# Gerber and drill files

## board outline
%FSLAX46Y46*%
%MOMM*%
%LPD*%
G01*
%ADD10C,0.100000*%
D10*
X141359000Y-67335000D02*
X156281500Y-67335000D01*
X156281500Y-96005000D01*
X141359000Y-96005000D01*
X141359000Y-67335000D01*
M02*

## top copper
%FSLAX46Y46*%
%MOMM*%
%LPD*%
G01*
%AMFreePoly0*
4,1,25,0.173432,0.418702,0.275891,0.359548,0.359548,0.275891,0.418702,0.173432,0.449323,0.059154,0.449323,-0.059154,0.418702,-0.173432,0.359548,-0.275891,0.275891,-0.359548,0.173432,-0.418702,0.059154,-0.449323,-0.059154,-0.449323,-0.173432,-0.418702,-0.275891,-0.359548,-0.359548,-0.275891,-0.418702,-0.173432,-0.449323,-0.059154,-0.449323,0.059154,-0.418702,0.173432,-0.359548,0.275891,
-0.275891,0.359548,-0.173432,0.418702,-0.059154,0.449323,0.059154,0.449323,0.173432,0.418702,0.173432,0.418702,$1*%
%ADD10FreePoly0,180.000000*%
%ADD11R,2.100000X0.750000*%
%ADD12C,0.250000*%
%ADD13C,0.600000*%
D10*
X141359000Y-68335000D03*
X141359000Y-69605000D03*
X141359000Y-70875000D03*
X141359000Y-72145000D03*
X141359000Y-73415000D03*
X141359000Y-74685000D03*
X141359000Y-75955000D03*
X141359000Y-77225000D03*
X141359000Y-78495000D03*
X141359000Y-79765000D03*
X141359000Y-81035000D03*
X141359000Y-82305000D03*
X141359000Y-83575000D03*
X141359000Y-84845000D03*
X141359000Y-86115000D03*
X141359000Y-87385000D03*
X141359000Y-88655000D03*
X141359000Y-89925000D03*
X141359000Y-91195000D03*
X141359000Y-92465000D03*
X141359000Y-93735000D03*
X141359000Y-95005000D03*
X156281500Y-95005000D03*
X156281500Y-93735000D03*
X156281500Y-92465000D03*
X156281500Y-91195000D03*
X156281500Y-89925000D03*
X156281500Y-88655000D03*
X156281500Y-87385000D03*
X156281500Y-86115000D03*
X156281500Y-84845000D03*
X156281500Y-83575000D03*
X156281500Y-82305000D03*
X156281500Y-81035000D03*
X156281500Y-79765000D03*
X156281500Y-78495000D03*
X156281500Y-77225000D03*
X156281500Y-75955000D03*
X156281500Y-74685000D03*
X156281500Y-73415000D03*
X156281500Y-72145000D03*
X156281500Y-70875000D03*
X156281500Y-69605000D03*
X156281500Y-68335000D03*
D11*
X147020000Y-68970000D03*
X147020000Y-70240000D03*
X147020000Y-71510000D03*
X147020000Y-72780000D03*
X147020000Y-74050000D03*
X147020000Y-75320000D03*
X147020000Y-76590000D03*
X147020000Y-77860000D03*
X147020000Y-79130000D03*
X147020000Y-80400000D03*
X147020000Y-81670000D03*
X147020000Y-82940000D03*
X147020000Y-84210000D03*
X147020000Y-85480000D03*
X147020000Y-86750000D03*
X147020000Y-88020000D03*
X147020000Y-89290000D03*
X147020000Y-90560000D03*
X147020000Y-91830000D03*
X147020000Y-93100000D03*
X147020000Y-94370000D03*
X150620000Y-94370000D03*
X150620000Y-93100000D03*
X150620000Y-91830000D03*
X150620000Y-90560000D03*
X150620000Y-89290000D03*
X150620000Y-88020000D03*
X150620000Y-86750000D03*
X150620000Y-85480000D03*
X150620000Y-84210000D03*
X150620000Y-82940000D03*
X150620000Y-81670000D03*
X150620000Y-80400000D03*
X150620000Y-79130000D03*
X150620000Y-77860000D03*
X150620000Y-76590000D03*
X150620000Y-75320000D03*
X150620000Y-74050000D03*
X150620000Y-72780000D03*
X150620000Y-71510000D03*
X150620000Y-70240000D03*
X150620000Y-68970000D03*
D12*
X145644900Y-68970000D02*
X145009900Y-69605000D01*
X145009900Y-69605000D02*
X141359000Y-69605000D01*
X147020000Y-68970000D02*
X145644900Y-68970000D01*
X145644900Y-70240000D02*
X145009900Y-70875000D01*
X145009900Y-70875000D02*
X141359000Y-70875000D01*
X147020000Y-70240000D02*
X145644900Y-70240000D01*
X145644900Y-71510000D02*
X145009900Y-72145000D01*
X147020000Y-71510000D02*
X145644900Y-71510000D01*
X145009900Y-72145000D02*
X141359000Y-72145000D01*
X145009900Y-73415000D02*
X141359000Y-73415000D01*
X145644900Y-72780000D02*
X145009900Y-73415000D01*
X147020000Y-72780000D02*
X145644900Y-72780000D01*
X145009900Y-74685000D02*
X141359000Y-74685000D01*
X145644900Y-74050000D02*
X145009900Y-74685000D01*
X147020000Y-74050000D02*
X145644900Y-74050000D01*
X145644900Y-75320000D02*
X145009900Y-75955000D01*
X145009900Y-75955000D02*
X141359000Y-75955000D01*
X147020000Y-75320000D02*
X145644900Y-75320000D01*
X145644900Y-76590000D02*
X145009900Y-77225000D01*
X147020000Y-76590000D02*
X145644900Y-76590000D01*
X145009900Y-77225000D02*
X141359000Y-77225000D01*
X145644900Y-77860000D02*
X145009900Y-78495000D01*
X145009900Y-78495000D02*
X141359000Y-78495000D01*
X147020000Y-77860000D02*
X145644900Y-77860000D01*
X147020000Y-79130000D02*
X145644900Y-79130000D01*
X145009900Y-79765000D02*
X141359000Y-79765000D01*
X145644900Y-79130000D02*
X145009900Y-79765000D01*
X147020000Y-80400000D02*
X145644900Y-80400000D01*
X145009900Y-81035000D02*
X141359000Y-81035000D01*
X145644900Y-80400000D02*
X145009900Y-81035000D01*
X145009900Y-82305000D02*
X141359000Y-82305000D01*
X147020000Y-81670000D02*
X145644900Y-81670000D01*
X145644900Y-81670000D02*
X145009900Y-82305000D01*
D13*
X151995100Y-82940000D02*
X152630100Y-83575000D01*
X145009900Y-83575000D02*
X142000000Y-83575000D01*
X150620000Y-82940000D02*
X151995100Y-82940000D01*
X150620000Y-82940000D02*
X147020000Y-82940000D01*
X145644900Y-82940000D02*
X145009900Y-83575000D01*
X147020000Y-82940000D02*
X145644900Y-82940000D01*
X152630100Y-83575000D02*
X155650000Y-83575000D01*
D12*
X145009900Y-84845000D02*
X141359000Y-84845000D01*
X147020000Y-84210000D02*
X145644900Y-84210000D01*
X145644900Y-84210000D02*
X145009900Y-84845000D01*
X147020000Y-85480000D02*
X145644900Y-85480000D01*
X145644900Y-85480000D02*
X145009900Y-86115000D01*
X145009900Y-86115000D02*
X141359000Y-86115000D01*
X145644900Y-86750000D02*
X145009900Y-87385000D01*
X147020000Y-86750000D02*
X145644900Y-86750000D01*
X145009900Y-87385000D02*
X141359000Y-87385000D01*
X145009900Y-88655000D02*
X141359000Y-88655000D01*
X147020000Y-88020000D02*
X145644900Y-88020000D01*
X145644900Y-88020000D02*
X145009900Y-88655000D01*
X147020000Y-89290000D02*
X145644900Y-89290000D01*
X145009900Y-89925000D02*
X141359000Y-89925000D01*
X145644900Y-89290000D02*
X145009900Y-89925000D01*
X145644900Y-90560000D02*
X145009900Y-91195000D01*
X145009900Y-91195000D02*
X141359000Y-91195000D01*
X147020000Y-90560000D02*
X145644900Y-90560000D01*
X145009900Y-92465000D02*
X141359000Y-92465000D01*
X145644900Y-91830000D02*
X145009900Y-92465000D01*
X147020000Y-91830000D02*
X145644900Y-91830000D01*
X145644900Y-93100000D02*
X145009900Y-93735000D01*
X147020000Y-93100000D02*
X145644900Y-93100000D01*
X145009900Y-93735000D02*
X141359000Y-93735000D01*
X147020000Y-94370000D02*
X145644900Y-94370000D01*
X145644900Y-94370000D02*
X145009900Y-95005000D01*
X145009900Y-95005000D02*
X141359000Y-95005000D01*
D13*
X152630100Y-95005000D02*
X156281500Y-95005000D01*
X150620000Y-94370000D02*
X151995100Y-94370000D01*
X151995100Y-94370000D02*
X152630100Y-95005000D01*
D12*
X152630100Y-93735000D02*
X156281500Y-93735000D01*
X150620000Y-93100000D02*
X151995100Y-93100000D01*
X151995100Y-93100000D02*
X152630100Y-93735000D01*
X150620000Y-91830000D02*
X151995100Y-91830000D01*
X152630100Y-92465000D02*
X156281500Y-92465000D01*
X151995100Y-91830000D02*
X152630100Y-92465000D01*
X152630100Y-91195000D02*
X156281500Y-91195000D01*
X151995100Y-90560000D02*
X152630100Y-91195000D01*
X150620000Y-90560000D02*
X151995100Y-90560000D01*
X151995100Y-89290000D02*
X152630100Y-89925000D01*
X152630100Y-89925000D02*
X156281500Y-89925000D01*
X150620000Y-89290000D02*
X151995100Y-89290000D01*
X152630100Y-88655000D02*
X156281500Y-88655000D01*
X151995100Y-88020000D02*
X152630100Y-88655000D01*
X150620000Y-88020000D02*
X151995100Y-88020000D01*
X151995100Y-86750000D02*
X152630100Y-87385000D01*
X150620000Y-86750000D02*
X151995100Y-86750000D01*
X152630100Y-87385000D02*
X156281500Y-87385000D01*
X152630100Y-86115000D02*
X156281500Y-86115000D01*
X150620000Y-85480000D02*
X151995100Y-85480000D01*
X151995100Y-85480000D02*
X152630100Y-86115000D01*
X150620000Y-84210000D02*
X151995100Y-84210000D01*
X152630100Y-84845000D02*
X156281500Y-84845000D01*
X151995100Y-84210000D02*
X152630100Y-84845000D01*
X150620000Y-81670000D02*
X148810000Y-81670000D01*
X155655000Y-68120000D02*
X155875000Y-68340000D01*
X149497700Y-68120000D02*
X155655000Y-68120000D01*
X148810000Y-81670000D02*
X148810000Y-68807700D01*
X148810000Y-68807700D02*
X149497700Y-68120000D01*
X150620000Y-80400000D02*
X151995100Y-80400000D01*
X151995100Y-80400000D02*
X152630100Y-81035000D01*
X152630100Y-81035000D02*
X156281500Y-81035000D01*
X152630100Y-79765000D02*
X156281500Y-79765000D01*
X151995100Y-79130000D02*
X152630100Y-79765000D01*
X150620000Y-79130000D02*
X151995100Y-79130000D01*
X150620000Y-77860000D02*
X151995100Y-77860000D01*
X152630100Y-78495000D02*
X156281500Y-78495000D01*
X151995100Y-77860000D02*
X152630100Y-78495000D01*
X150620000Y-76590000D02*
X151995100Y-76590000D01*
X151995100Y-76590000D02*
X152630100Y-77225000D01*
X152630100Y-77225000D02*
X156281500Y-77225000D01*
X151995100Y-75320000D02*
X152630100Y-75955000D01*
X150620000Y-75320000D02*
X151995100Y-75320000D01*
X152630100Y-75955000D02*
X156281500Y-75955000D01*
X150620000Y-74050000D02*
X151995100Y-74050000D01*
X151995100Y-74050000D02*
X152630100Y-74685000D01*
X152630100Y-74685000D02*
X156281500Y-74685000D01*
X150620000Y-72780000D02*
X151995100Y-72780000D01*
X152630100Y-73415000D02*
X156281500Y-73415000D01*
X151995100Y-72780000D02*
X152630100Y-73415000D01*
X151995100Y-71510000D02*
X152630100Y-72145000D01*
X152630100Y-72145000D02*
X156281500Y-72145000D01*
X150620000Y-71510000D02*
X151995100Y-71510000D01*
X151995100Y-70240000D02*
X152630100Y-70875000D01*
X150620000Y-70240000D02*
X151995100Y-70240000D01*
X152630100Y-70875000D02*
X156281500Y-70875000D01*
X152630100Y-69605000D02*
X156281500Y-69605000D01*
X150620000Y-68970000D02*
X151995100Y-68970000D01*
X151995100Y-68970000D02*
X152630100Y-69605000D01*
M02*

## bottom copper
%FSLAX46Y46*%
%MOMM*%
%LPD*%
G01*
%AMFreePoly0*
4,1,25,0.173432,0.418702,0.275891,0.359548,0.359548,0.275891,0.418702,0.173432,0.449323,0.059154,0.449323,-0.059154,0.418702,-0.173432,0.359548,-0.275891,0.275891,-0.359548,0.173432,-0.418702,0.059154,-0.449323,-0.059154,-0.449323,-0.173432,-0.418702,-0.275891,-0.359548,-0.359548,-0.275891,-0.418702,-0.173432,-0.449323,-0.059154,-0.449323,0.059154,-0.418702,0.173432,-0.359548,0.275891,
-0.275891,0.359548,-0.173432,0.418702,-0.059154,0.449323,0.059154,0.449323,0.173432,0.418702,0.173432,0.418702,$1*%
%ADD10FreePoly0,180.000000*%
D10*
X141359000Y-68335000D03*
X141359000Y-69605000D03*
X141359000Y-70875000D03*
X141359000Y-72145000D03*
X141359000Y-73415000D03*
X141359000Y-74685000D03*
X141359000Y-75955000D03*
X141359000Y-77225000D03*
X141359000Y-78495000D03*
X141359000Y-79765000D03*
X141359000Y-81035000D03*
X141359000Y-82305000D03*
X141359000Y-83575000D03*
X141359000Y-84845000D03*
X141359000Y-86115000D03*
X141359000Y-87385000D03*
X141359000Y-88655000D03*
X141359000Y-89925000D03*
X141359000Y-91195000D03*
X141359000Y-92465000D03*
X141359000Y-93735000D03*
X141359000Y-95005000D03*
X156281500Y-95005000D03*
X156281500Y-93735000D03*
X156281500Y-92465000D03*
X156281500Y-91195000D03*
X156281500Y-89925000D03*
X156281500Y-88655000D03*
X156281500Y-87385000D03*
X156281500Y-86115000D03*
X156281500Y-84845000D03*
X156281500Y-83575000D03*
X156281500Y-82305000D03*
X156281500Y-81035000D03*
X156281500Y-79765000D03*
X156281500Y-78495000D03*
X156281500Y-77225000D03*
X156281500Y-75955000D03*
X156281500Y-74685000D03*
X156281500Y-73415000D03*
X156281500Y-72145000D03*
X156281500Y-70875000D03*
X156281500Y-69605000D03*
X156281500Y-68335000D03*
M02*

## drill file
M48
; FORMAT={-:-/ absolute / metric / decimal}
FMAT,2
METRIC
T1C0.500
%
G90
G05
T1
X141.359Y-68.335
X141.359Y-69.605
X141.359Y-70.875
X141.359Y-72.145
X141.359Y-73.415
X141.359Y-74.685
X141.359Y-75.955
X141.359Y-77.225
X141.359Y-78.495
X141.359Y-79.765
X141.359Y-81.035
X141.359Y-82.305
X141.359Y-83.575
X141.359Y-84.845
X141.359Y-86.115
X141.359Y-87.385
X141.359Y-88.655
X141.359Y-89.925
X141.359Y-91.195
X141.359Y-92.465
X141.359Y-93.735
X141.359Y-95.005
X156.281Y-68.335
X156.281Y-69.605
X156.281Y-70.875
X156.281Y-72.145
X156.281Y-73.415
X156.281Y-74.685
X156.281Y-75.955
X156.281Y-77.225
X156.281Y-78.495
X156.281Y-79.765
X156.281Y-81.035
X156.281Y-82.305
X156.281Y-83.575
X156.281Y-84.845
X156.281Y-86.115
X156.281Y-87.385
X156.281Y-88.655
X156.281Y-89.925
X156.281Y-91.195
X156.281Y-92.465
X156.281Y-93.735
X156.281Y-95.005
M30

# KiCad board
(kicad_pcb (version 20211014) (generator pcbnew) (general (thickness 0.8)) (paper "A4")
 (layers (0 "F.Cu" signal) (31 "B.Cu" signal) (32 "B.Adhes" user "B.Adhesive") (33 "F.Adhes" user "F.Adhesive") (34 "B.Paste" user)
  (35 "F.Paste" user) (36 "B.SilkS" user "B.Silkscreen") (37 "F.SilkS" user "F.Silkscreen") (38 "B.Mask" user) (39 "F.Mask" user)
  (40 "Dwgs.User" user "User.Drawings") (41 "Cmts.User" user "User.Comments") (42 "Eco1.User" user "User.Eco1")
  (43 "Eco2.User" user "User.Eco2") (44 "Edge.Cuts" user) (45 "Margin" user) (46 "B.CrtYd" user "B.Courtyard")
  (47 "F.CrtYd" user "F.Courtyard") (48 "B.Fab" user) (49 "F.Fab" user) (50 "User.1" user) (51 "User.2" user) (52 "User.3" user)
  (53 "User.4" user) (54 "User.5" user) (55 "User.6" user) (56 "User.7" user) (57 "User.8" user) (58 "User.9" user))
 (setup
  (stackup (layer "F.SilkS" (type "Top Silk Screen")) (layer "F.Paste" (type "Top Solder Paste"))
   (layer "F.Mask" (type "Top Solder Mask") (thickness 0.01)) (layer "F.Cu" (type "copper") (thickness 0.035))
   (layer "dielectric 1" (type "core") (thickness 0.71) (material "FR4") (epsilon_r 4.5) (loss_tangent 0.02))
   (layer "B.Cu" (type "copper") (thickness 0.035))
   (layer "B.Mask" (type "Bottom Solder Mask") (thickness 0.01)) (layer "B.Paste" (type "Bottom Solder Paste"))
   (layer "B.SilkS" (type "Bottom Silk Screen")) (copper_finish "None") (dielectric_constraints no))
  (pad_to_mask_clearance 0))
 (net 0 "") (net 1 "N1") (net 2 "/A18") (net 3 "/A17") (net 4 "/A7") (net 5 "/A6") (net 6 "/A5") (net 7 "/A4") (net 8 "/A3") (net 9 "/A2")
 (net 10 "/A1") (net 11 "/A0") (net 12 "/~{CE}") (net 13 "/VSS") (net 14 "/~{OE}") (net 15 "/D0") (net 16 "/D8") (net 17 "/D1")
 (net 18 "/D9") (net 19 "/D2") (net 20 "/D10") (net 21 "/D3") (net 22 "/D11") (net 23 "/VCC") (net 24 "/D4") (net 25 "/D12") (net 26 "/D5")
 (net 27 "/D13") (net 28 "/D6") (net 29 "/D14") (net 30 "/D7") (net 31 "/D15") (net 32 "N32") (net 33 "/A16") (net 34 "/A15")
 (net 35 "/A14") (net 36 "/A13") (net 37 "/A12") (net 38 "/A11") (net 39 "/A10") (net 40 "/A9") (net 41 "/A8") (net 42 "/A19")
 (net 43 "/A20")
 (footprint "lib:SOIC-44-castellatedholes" (layer "F.Cu") (at 148.82 81.67)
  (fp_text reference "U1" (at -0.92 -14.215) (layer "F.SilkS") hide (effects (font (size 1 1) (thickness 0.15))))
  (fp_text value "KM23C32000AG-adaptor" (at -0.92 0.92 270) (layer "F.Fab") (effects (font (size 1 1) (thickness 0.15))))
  (pad "1" thru_hole custom (at -7.461 -13.335 180) (size 0.9064 0.9064) (drill 0.5) (layers *.Cu *.Mask) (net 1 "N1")
   (solder_mask_margin 0.0762) (options (clearance outline) (anchor circle)) (primitives))
  (pad "2" thru_hole custom (at -7.461 -12.065 180) (size 0.9064 0.9064) (drill 0.5) (layers *.Cu *.Mask) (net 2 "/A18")
   (solder_mask_margin 0.0762) (options (clearance outline) (anchor circle)) (primitives))
  (pad "3" thru_hole custom (at -7.461 -10.795 180) (size 0.9064 0.9064) (drill 0.5) (layers *.Cu *.Mask) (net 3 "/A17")
   (solder_mask_margin 0.0762) (options (clearance outline) (anchor circle)) (primitives))
  (pad "4" thru_hole custom (at -7.461 -9.525 180) (size 0.9064 0.9064) (drill 0.5) (layers *.Cu *.Mask) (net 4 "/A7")
   (solder_mask_margin 0.0762) (options (clearance outline) (anchor circle)) (primitives))
  (pad "5" thru_hole custom (at -7.461 -8.255 180) (size 0.9064 0.9064) (drill 0.5) (layers *.Cu *.Mask) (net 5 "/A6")
   (solder_mask_margin 0.0762) (options (clearance outline) (anchor circle)) (primitives))
  (pad "6" thru_hole custom (at -7.461 -6.985 180) (size 0.9064 0.9064) (drill 0.5) (layers *.Cu *.Mask) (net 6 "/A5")
   (solder_mask_margin 0.0762) (options (clearance outline) (anchor circle)) (primitives))
  (pad "7" thru_hole custom (at -7.461 -5.715 180) (size 0.9064 0.9064) (drill 0.5) (layers *.Cu *.Mask) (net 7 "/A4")
   (solder_mask_margin 0.0762) (options (clearance outline) (anchor circle)) (primitives))
  (pad "8" thru_hole custom (at -7.461 -4.445 180) (size 0.9064 0.9064) (drill 0.5) (layers *.Cu *.Mask) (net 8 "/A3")
   (solder_mask_margin 0.0762) (options (clearance outline) (anchor circle)) (primitives))
  (pad "9" thru_hole custom (at -7.461 -3.175 180) (size 0.9064 0.9064) (drill 0.5) (layers *.Cu *.Mask) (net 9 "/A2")
   (solder_mask_margin 0.0762) (options (clearance outline) (anchor circle)) (primitives))
  (pad "10" thru_hole custom (at -7.461 -1.905 180) (size 0.9064 0.9064) (drill 0.5) (layers *.Cu *.Mask) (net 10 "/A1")
   (solder_mask_margin 0.0762) (options (clearance outline) (anchor circle)) (primitives))
  (pad "11" thru_hole custom (at -7.461 -0.635 180) (size 0.9064 0.9064) (drill 0.5) (layers *.Cu *.Mask) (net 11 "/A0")
   (solder_mask_margin 0.0762) (options (clearance outline) (anchor circle)) (primitives))
  (pad "12" thru_hole custom (at -7.461 0.635 180) (size 0.9064 0.9064) (drill 0.5) (layers *.Cu *.Mask) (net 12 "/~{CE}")
   (solder_mask_margin 0.0762) (options (clearance outline) (anchor circle)) (primitives))
  (pad "13" thru_hole custom (at -7.461 1.905 180) (size 0.9064 0.9064) (drill 0.5) (layers *.Cu *.Mask) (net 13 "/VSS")
   (solder_mask_margin 0.0762) (options (clearance outline) (anchor circle)) (primitives))
  (pad "14" thru_hole custom (at -7.461 3.175 180) (size 0.9064 0.9064) (drill 0.5) (layers *.Cu *.Mask) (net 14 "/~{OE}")
   (solder_mask_margin 0.0762) (options (clearance outline) (anchor circle)) (primitives))
  (pad "15" thru_hole custom (at -7.461 4.445 180) (size 0.9064 0.9064) (drill 0.5) (layers *.Cu *.Mask) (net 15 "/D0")
   (solder_mask_margin 0.0762) (options (clearance outline) (anchor circle)) (primitives))
  (pad "16" thru_hole custom (at -7.461 5.715 180) (size 0.9064 0.9064) (drill 0.5) (layers *.Cu *.Mask) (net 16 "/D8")
   (solder_mask_margin 0.0762) (options (clearance outline) (anchor circle)) (primitives))
  (pad "17" thru_hole custom (at -7.461 6.985 180) (size 0.9064 0.9064) (drill 0.5) (layers *.Cu *.Mask) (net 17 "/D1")
   (solder_mask_margin 0.0762) (options (clearance outline) (anchor circle)) (primitives))
  (pad "18" thru_hole custom (at -7.461 8.255 180) (size 0.9064 0.9064) (drill 0.5) (layers *.Cu *.Mask) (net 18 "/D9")
   (solder_mask_margin 0.0762) (options (clearance outline) (anchor circle)) (primitives))
  (pad "19" thru_hole custom (at -7.461 9.525 180) (size 0.9064 0.9064) (drill 0.5) (layers *.Cu *.Mask) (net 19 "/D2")
   (solder_mask_margin 0.0762) (options (clearance outline) (anchor circle)) (primitives))
  (pad "20" thru_hole custom (at -7.461 10.795 180) (size 0.9064 0.9064) (drill 0.5) (layers *.Cu *.Mask) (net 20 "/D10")
   (solder_mask_margin 0.0762) (options (clearance outline) (anchor circle)) (primitives))
  (pad "21" thru_hole custom (at -7.461 12.065 180) (size 0.9064 0.9064) (drill 0.5) (layers *.Cu *.Mask) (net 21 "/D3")
   (solder_mask_margin 0.0762) (options (clearance outline) (anchor circle)) (primitives))
  (pad "22" thru_hole custom (at -7.461 13.335 180) (size 0.9064 0.9064) (drill 0.5) (layers *.Cu *.Mask) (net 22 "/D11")
   (solder_mask_margin 0.0762) (options (clearance outline) (anchor circle)) (primitives))
  (pad "23" thru_hole custom (at 7.4615 13.335 180) (size 0.9064 0.9064) (drill 0.5) (layers *.Cu *.Mask) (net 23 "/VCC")
   (solder_mask_margin 0.0762) (options (clearance outline) (anchor circle)) (primitives))
  (pad "24" thru_hole custom (at 7.4615 12.065 180) (size 0.9064 0.9064) (drill 0.5) (layers *.Cu *.Mask) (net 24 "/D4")
   (solder_mask_margin 0.0762) (options (clearance outline) (anchor circle)) (primitives))
  (pad "25" thru_hole custom (at 7.4615 10.795 180) (size 0.9064 0.9064) (drill 0.5) (layers *.Cu *.Mask) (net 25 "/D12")
   (solder_mask_margin 0.0762) (options (clearance outline) (anchor circle)) (primitives))
  (pad "26" thru_hole custom (at 7.4615 9.525 180) (size 0.9064 0.9064) (drill 0.5) (layers *.Cu *.Mask) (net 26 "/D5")
   (solder_mask_margin 0.0762) (options (clearance outline) (anchor circle)) (primitives))
  (pad "27" thru_hole custom (at 7.4615 8.255 180) (size 0.9064 0.9064) (drill 0.5) (layers *.Cu *.Mask) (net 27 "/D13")
   (solder_mask_margin 0.0762) (options (clearance outline) (anchor circle)) (primitives))
  (pad "28" thru_hole custom (at 7.4615 6.985 180) (size 0.9064 0.9064) (drill 0.5) (layers *.Cu *.Mask) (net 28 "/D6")
   (solder_mask_margin 0.0762) (options (clearance outline) (anchor circle)) (primitives))
  (pad "29" thru_hole custom (at 7.4615 5.715 180) (size 0.9064 0.9064) (drill 0.5) (layers *.Cu *.Mask) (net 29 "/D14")
   (solder_mask_margin 0.0762) (options (clearance outline) (anchor circle)) (primitives))
  (pad "30" thru_hole custom (at 7.4615 4.445 180) (size 0.9064 0.9064) (drill 0.5) (layers *.Cu *.Mask) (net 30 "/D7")
   (solder_mask_margin 0.0762) (options (clearance outline) (anchor circle)) (primitives))
  (pad "31" thru_hole custom (at 7.4615 3.175 180) (size 0.9064 0.9064) (drill 0.5) (layers *.Cu *.Mask) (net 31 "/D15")
   (solder_mask_margin 0.0762) (options (clearance outline) (anchor circle)) (primitives))
  (pad "32" thru_hole custom (at 7.4615 1.905 180) (size 0.9064 0.9064) (drill 0.5) (layers *.Cu *.Mask) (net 13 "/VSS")
   (solder_mask_margin 0.0762) (options (clearance outline) (anchor circle)) (primitives))
  (pad "33" thru_hole custom (at 7.4615 0.635 180) (size 0.9064 0.9064) (drill 0.5) (layers *.Cu *.Mask) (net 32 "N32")
   (solder_mask_margin 0.0762) (options (clearance outline) (anchor circle)) (primitives))
  (pad "34" thru_hole custom (at 7.4615 -0.635 180) (size 0.9064 0.9064) (drill 0.5) (layers *.Cu *.Mask) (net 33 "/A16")
   (solder_mask_margin 0.0762) (options (clearance outline) (anchor circle)) (primitives))
  (pad "35" thru_hole custom (at 7.4615 -1.905 180) (size 0.9064 0.9064) (drill 0.5) (layers *.Cu *.Mask) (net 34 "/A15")
   (solder_mask_margin 0.0762) (options (clearance outline) (anchor circle)) (primitives))
  (pad "36" thru_hole custom (at 7.4615 -3.175 180) (size 0.9064 0.9064) (drill 0.5) (layers *.Cu *.Mask) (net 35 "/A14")
   (solder_mask_margin 0.0762) (options (clearance outline) (anchor circle)) (primitives))
  (pad "37" thru_hole custom (at 7.4615 -4.445 180) (size 0.9064 0.9064) (drill 0.5) (layers *.Cu *.Mask) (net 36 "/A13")
   (solder_mask_margin 0.0762) (options (clearance outline) (anchor circle)) (primitives))
  (pad "38" thru_hole custom (at 7.4615 -5.715 180) (size 0.9064 0.9064) (drill 0.5) (layers *.Cu *.Mask) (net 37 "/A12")
   (solder_mask_margin 0.0762) (options (clearance outline) (anchor circle)) (primitives))
  (pad "39" thru_hole custom (at 7.4615 -6.985 180) (size 0.9064 0.9064) (drill 0.5) (layers *.Cu *.Mask) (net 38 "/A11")
   (solder_mask_margin 0.0762) (options (clearance outline) (anchor circle)) (primitives))
  (pad "40" thru_hole custom (at 7.4615 -8.255 180) (size 0.9064 0.9064) (drill 0.5) (layers *.Cu *.Mask) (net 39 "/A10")
   (solder_mask_margin 0.0762) (options (clearance outline) (anchor circle)) (primitives))
  (pad "41" thru_hole custom (at 7.4615 -9.525 180) (size 0.9064 0.9064) (drill 0.5) (layers *.Cu *.Mask) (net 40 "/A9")
   (solder_mask_margin 0.0762) (options (clearance outline) (anchor circle)) (primitives))
  (pad "42" thru_hole custom (at 7.4615 -10.795 180) (size 0.9064 0.9064) (drill 0.5) (layers *.Cu *.Mask) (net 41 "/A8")
   (solder_mask_margin 0.0762) (options (clearance outline) (anchor circle)) (primitives))
  (pad "43" thru_hole custom (at 7.4615 -12.065 180) (size 0.9064 0.9064) (drill 0.5) (layers *.Cu *.Mask) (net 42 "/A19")
   (solder_mask_margin 0.0762) (options (clearance outline) (anchor circle)) (primitives))
  (pad "44" thru_hole custom (at 7.4615 -13.335 180) (size 0.9064 0.9064) (drill 0.5) (layers *.Cu *.Mask) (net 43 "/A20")
   (solder_mask_margin 0.0762) (options (clearance outline) (anchor circle)) (primitives)))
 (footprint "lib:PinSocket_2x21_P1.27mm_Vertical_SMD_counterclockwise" (layer "F.Cu") (at 148.82 81.67)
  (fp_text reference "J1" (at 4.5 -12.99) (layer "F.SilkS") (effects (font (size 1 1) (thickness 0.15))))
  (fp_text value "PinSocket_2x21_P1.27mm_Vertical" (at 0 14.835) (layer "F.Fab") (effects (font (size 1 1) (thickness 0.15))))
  (pad "1" smd rect (at -1.8 -12.7) (size 2.1 0.75) (layers "F.Cu" "F.Paste" "F.Mask") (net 2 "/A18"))
  (pad "2" smd rect (at -1.8 -11.43) (size 2.1 0.75) (layers "F.Cu" "F.Paste" "F.Mask") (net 3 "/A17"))
  (pad "3" smd rect (at -1.8 -10.16) (size 2.1 0.75) (layers "F.Cu" "F.Paste" "F.Mask") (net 4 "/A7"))
  (pad "4" smd rect (at -1.8 -8.89) (size 2.1 0.75) (layers "F.Cu" "F.Paste" "F.Mask") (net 5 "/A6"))
  (pad "5" smd rect (at -1.8 -7.62) (size 2.1 0.75) (layers "F.Cu" "F.Paste" "F.Mask") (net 6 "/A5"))
  (pad "6" smd rect (at -1.8 -6.35) (size 2.1 0.75) (layers "F.Cu" "F.Paste" "F.Mask") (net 7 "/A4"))
  (pad "7" smd rect (at -1.8 -5.08) (size 2.1 0.75) (layers "F.Cu" "F.Paste" "F.Mask") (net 8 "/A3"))
  (pad "8" smd rect (at -1.8 -3.81) (size 2.1 0.75) (layers "F.Cu" "F.Paste" "F.Mask") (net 9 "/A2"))
  (pad "9" smd rect (at -1.8 -2.54) (size 2.1 0.75) (layers "F.Cu" "F.Paste" "F.Mask") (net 10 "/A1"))
  (pad "10" smd rect (at -1.8 -1.27) (size 2.1 0.75) (layers "F.Cu" "F.Paste" "F.Mask") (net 11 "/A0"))
  (pad "11" smd rect (at -1.8 0) (size 2.1 0.75) (layers "F.Cu" "F.Paste" "F.Mask") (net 12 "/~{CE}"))
  (pad "12" smd rect (at -1.8 1.27) (size 2.1 0.75) (layers "F.Cu" "F.Paste" "F.Mask") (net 13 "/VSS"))
  (pad "13" smd rect (at -1.8 2.54) (size 2.1 0.75) (layers "F.Cu" "F.Paste" "F.Mask") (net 14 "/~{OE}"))
  (pad "14" smd rect (at -1.8 3.81) (size 2.1 0.75) (layers "F.Cu" "F.Paste" "F.Mask") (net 15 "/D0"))
  (pad "15" smd rect (at -1.8 5.08) (size 2.1 0.75) (layers "F.Cu" "F.Paste" "F.Mask") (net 16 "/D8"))
  (pad "16" smd rect (at -1.8 6.35) (size 2.1 0.75) (layers "F.Cu" "F.Paste" "F.Mask") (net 17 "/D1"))
  (pad "17" smd rect (at -1.8 7.62) (size 2.1 0.75) (layers "F.Cu" "F.Paste" "F.Mask") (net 18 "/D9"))
  (pad "18" smd rect (at -1.8 8.89) (size 2.1 0.75) (layers "F.Cu" "F.Paste" "F.Mask") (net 19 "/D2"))
  (pad "19" smd rect (at -1.8 10.16) (size 2.1 0.75) (layers "F.Cu" "F.Paste" "F.Mask") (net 20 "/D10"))
  (pad "20" smd rect (at -1.8 11.43) (size 2.1 0.75) (layers "F.Cu" "F.Paste" "F.Mask") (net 21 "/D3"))
  (pad "21" smd rect (at -1.8 12.7) (size 2.1 0.75) (layers "F.Cu" "F.Paste" "F.Mask") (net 22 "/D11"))
  (pad "22" smd rect (at 1.8 12.7) (size 2.1 0.75) (layers "F.Cu" "F.Paste" "F.Mask") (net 23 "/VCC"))
  (pad "23" smd rect (at 1.8 11.43) (size 2.1 0.75) (layers "F.Cu" "F.Paste" "F.Mask") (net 24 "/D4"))
  (pad "24" smd rect (at 1.8 10.16) (size 2.1 0.75) (layers "F.Cu" "F.Paste" "F.Mask") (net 25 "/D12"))
  (pad "25" smd rect (at 1.8 8.89) (size 2.1 0.75) (layers "F.Cu" "F.Paste" "F.Mask") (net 26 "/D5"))
  (pad "26" smd rect (at 1.8 7.62) (size 2.1 0.75) (layers "F.Cu" "F.Paste" "F.Mask") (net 27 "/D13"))
  (pad "27" smd rect (at 1.8 6.35) (size 2.1 0.75) (layers "F.Cu" "F.Paste" "F.Mask") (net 28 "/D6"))
  (pad "28" smd rect (at 1.8 5.08) (size 2.1 0.75) (layers "F.Cu" "F.Paste" "F.Mask") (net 29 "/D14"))
  (pad "29" smd rect (at 1.8 3.81) (size 2.1 0.75) (layers "F.Cu" "F.Paste" "F.Mask") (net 30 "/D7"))
  (pad "30" smd rect (at 1.8 2.54) (size 2.1 0.75) (layers "F.Cu" "F.Paste" "F.Mask") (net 31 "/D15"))
  (pad "31" smd rect (at 1.8 1.27) (size 2.1 0.75) (layers "F.Cu" "F.Paste" "F.Mask") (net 13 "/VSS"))
  (pad "32" smd rect (at 1.8 0) (size 2.1 0.75) (layers "F.Cu" "F.Paste" "F.Mask") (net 43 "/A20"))
  (pad "33" smd rect (at 1.8 -1.27) (size 2.1 0.75) (layers "F.Cu" "F.Paste" "F.Mask") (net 33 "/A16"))
  (pad "34" smd rect (at 1.8 -2.54) (size 2.1 0.75) (layers "F.Cu" "F.Paste" "F.Mask") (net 34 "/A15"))
  (pad "35" smd rect (at 1.8 -3.81) (size 2.1 0.75) (layers "F.Cu" "F.Paste" "F.Mask") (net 35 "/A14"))
  (pad "36" smd rect (at 1.8 -5.08) (size 2.1 0.75) (layers "F.Cu" "F.Paste" "F.Mask") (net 36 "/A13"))
  (pad "37" smd rect (at 1.8 -6.35) (size 2.1 0.75) (layers "F.Cu" "F.Paste" "F.Mask") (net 37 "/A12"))
  (pad "38" smd rect (at 1.8 -7.62) (size 2.1 0.75) (layers "F.Cu" "F.Paste" "F.Mask") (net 38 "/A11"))
  (pad "39" smd rect (at 1.8 -8.89) (size 2.1 0.75) (layers "F.Cu" "F.Paste" "F.Mask") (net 39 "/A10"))
  (pad "40" smd rect (at 1.8 -10.16) (size 2.1 0.75) (layers "F.Cu" "F.Paste" "F.Mask") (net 40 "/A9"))
  (pad "41" smd rect (at 1.8 -11.43) (size 2.1 0.75) (layers "F.Cu" "F.Paste" "F.Mask") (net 41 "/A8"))
  (pad "42" smd rect (at 1.8 -12.7) (size 2.1 0.75) (layers "F.Cu" "F.Paste" "F.Mask") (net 42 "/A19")))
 (gr_rect (start 141.359 67.335) (end 156.2815 96.005) (layer "Edge.Cuts") (width 0.1) (fill none))
 (segment (start 145.6449 68.97) (end 145.0099 69.605) (width 0.25) (layer "F.Cu") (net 2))
 (segment (start 145.0099 69.605) (end 141.359 69.605) (width 0.25) (layer "F.Cu") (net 2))
 (segment (start 147.02 68.97) (end 145.6449 68.97) (width 0.25) (layer "F.Cu") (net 2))
 (segment (start 145.6449 70.24) (end 145.0099 70.875) (width 0.25) (layer "F.Cu") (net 3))
 (segment (start 145.0099 70.875) (end 141.359 70.875) (width 0.25) (layer "F.Cu") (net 3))
 (segment (start 147.02 70.24) (end 145.6449 70.24) (width 0.25) (layer "F.Cu") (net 3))
 (segment (start 145.6449 71.51) (end 145.0099 72.145) (width 0.25) (layer "F.Cu") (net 4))
 (segment (start 147.02 71.51) (end 145.6449 71.51) (width 0.25) (layer "F.Cu") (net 4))
 (segment (start 145.0099 72.145) (end 141.359 72.145) (width 0.25) (layer "F.Cu") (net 4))
 (segment (start 145.0099 73.415) (end 141.359 73.415) (width 0.25) (layer "F.Cu") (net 5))
 (segment (start 145.6449 72.78) (end 145.0099 73.415) (width 0.25) (layer "F.Cu") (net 5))
 (segment (start 147.02 72.78) (end 145.6449 72.78) (width 0.25) (layer "F.Cu") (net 5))
 (segment (start 145.0099 74.685) (end 141.359 74.685) (width 0.25) (layer "F.Cu") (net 6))
 (segment (start 145.6449 74.05) (end 145.0099 74.685) (width 0.25) (layer "F.Cu") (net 6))
 (segment (start 147.02 74.05) (end 145.6449 74.05) (width 0.25) (layer "F.Cu") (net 6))
 (segment (start 145.6449 75.32) (end 145.0099 75.955) (width 0.25) (layer "F.Cu") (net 7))
 (segment (start 145.0099 75.955) (end 141.359 75.955) (width 0.25) (layer "F.Cu") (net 7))
 (segment (start 147.02 75.32) (end 145.6449 75.32) (width 0.25) (layer "F.Cu") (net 7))
 (segment (start 145.6449 76.59) (end 145.0099 77.225) (width 0.25) (layer "F.Cu") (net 8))
 (segment (start 147.02 76.59) (end 145.6449 76.59) (width 0.25) (layer "F.Cu") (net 8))
 (segment (start 145.0099 77.225) (end 141.359 77.225) (width 0.25) (layer "F.Cu") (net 8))
 (segment (start 145.6449 77.86) (end 145.0099 78.495) (width 0.25) (layer "F.Cu") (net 9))
 (segment (start 145.0099 78.495) (end 141.359 78.495) (width 0.25) (layer "F.Cu") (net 9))
 (segment (start 147.02 77.86) (end 145.6449 77.86) (width 0.25) (layer "F.Cu") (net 9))
 (segment (start 147.02 79.13) (end 145.6449 79.13) (width 0.25) (layer "F.Cu") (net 10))
 (segment (start 145.0099 79.765) (end 141.359 79.765) (width 0.25) (layer "F.Cu") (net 10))
 (segment (start 145.6449 79.13) (end 145.0099 79.765) (width 0.25) (layer "F.Cu") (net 10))
 (segment (start 147.02 80.4) (end 145.6449 80.4) (width 0.25) (layer "F.Cu") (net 11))
 (segment (start 145.0099 81.035) (end 141.359 81.035) (width 0.25) (layer "F.Cu") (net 11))
 (segment (start 145.6449 80.4) (end 145.0099 81.035) (width 0.25) (layer "F.Cu") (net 11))
 (segment (start 145.0099 82.305) (end 141.359 82.305) (width 0.25) (layer "F.Cu") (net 12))
 (segment (start 147.02 81.67) (end 145.6449 81.67) (width 0.25) (layer "F.Cu") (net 12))
 (segment (start 145.6449 81.67) (end 145.0099 82.305) (width 0.25) (layer "F.Cu") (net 12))
 (segment (start 151.9951 82.94) (end 152.6301 83.575) (width 0.6) (layer "F.Cu") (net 13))
 (segment (start 145.0099 83.575) (end 142 83.575) (width 0.6) (layer "F.Cu") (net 13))
 (segment (start 150.62 82.94) (end 151.9951 82.94) (width 0.6) (layer "F.Cu") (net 13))
 (segment (start 150.62 82.94) (end 147.02 82.94) (width 0.6) (layer "F.Cu") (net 13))
 (segment (start 145.6449 82.94) (end 145.0099 83.575) (width 0.6) (layer "F.Cu") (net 13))
 (segment (start 147.02 82.94) (end 145.6449 82.94) (width 0.6) (layer "F.Cu") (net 13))
 (segment (start 152.6301 83.575) (end 155.65 83.575) (width 0.6) (layer "F.Cu") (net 13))
 (segment (start 145.0099 84.845) (end 141.359 84.845) (width 0.25) (layer "F.Cu") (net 14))
 (segment (start 147.02 84.21) (end 145.6449 84.21) (width 0.25) (layer "F.Cu") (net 14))
 (segment (start 145.6449 84.21) (end 145.0099 84.845) (width 0.25) (layer "F.Cu") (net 14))
 (segment (start 147.02 85.48) (end 145.6449 85.48) (width 0.25) (layer "F.Cu") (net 15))
 (segment (start 145.6449 85.48) (end 145.0099 86.115) (width 0.25) (layer "F.Cu") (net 15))
 (segment (start 145.0099 86.115) (end 141.359 86.115) (width 0.25) (layer "F.Cu") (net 15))
 (segment (start 145.6449 86.75) (end 145.0099 87.385) (width 0.25) (layer "F.Cu") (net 16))
 (segment (start 147.02 86.75) (end 145.6449 86.75) (width 0.25) (layer "F.Cu") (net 16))
 (segment (start 145.0099 87.385) (end 141.359 87.385) (width 0.25) (layer "F.Cu") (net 16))
 (segment (start 145.0099 88.655) (end 141.359 88.655) (width 0.25) (layer "F.Cu") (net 17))
 (segment (start 147.02 88.02) (end 145.6449 88.02) (width 0.25) (layer "F.Cu") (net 17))
 (segment (start 145.6449 88.02) (end 145.0099 88.655) (width 0.25) (layer "F.Cu") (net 17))
 (segment (start 147.02 89.29) (end 145.6449 89.29) (width 0.25) (layer "F.Cu") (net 18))
 (segment (start 145.0099 89.925) (end 141.359 89.925) (width 0.25) (layer "F.Cu") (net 18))
 (segment (start 145.6449 89.29) (end 145.0099 89.925) (width 0.25) (layer "F.Cu") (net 18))
 (segment (start 145.6449 90.56) (end 145.0099 91.195) (width 0.25) (layer "F.Cu") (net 19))
 (segment (start 145.0099 91.195) (end 141.359 91.195) (width 0.25) (layer "F.Cu") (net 19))
 (segment (start 147.02 90.56) (end 145.6449 90.56) (width 0.25) (layer "F.Cu") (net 19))
 (segment (start 145.0099 92.465) (end 141.359 92.465) (width 0.25) (layer "F.Cu") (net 20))
 (segment (start 145.6449 91.83) (end 145.0099 92.465) (width 0.25) (layer "F.Cu") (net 20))
 (segment (start 147.02 91.83) (end 145.6449 91.83) (width 0.25) (layer "F.Cu") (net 20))
 (segment (start 145.6449 93.1) (end 145.0099 93.735) (width 0.25) (layer "F.Cu") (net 21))
 (segment (start 147.02 93.1) (end 145.6449 93.1) (width 0.25) (layer "F.Cu") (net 21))
 (segment (start 145.0099 93.735) (end 141.359 93.735) (width 0.25) (layer "F.Cu") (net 21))
 (segment (start 147.02 94.37) (end 145.6449 94.37) (width 0.25) (layer "F.Cu") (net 22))
 (segment (start 145.6449 94.37) (end 145.0099 95.005) (width 0.25) (layer "F.Cu") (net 22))
 (segment (start 145.0099 95.005) (end 141.359 95.005) (width 0.25) (layer "F.Cu") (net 22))
 (segment (start 152.6301 95.005) (end 156.2815 95.005) (width 0.6) (layer "F.Cu") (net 23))
 (segment (start 150.62 94.37) (end 151.9951 94.37) (width 0.6) (layer "F.Cu") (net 23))
 (segment (start 151.9951 94.37) (end 152.6301 95.005) (width 0.6) (layer "F.Cu") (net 23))
 (segment (start 152.6301 93.735) (end 156.2815 93.735) (width 0.25) (layer "F.Cu") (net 24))
 (segment (start 150.62 93.1) (end 151.9951 93.1) (width 0.25) (layer "F.Cu") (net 24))
 (segment (start 151.9951 93.1) (end 152.6301 93.735) (width 0.25) (layer "F.Cu") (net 24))
 (segment (start 150.62 91.83) (end 151.9951 91.83) (width 0.25) (layer "F.Cu") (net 25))
 (segment (start 152.6301 92.465) (end 156.2815 92.465) (width 0.25) (layer "F.Cu") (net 25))
 (segment (start 151.9951 91.83) (end 152.6301 92.465) (width 0.25) (layer "F.Cu") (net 25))
 (segment (start 152.6301 91.195) (end 156.2815 91.195) (width 0.25) (layer "F.Cu") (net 26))
 (segment (start 151.9951 90.56) (end 152.6301 91.195) (width 0.25) (layer "F.Cu") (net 26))
 (segment (start 150.62 90.56) (end 151.9951 90.56) (width 0.25) (layer "F.Cu") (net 26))
 (segment (start 151.9951 89.29) (end 152.6301 89.925) (width 0.25) (layer "F.Cu") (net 27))
 (segment (start 152.6301 89.925) (end 156.2815 89.925) (width 0.25) (layer "F.Cu") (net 27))
 (segment (start 150.62 89.29) (end 151.9951 89.29) (width 0.25) (layer "F.Cu") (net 27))
 (segment (start 152.6301 88.655) (end 156.2815 88.655) (width 0.25) (layer "F.Cu") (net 28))
 (segment (start 151.9951 88.02) (end 152.6301 88.655) (width 0.25) (layer "F.Cu") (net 28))
 (segment (start 150.62 88.02) (end 151.9951 88.02) (width 0.25) (layer "F.Cu") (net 28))
 (segment (start 151.9951 86.75) (end 152.6301 87.385) (width 0.25) (layer "F.Cu") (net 29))
 (segment (start 150.62 86.75) (end 151.9951 86.75) (width 0.25) (layer "F.Cu") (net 29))
 (segment (start 152.6301 87.385) (end 156.2815 87.385) (width 0.25) (layer "F.Cu") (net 29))
 (segment (start 152.6301 86.115) (end 156.2815 86.115) (width 0.25) (layer "F.Cu") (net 30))
 (segment (start 150.62 85.48) (end 151.9951 85.48) (width 0.25) (layer "F.Cu") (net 30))
 (segment (start 151.9951 85.48) (end 152.6301 86.115) (width 0.25) (layer "F.Cu") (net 30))
 (segment (start 150.62 84.21) (end 151.9951 84.21) (width 0.25) (layer "F.Cu") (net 31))
 (segment (start 152.6301 84.845) (end 156.2815 84.845) (width 0.25) (layer "F.Cu") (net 31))
 (segment (start 151.9951 84.21) (end 152.6301 84.845) (width 0.25) (layer "F.Cu") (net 31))
 (segment (start 150.62 81.67) (end 148.81 81.67) (width 0.25) (layer "F.Cu") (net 43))
 (segment (start 155.655 68.12) (end 155.875 68.34) (width 0.25) (layer "F.Cu") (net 43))
 (segment (start 149.4977 68.12) (end 155.655 68.12) (width 0.25) (layer "F.Cu") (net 43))
 (segment (start 148.81 81.67) (end 148.81 68.8077) (width 0.25) (layer "F.Cu") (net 43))
 (segment (start 148.81 68.8077) (end 149.4977 68.12) (width 0.25) (layer "F.Cu") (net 43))
 (segment (start 150.62 80.4) (end 151.9951 80.4) (width 0.25) (layer "F.Cu") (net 33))
 (segment (start 151.9951 80.4) (end 152.6301 81.035) (width 0.25) (layer "F.Cu") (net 33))
 (segment (start 152.6301 81.035) (end 156.2815 81.035) (width 0.25) (layer "F.Cu") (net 33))
 (segment (start 152.6301 79.765) (end 156.2815 79.765) (width 0.25) (layer "F.Cu") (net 34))
 (segment (start 151.9951 79.13) (end 152.6301 79.765) (width 0.25) (layer "F.Cu") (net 34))
 (segment (start 150.62 79.13) (end 151.9951 79.13) (width 0.25) (layer "F.Cu") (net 34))
 (segment (start 150.62 77.86) (end 151.9951 77.86) (width 0.25) (layer "F.Cu") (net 35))
 (segment (start 152.6301 78.495) (end 156.2815 78.495) (width 0.25) (layer "F.Cu") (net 35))
 (segment (start 151.9951 77.86) (end 152.6301 78.495) (width 0.25) (layer "F.Cu") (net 35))
 (segment (start 150.62 76.59) (end 151.9951 76.59) (width 0.25) (layer "F.Cu") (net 36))
 (segment (start 151.9951 76.59) (end 152.6301 77.225) (width 0.25) (layer "F.Cu") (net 36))
 (segment (start 152.6301 77.225) (end 156.2815 77.225) (width 0.25) (layer "F.Cu") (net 36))
 (segment (start 151.9951 75.32) (end 152.6301 75.955) (width 0.25) (layer "F.Cu") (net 37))
 (segment (start 150.62 75.32) (end 151.9951 75.32) (width 0.25) (layer "F.Cu") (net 37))
 (segment (start 152.6301 75.955) (end 156.2815 75.955) (width 0.25) (layer "F.Cu") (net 37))
 (segment (start 150.62 74.05) (end 151.9951 74.05) (width 0.25) (layer "F.Cu") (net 38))
 (segment (start 151.9951 74.05) (end 152.6301 74.685) (width 0.25) (layer "F.Cu") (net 38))
 (segment (start 152.6301 74.685) (end 156.2815 74.685) (width 0.25) (layer "F.Cu") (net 38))
 (segment (start 150.62 72.78) (end 151.9951 72.78) (width 0.25) (layer "F.Cu") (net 39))
 (segment (start 152.6301 73.415) (end 156.2815 73.415) (width 0.25) (layer "F.Cu") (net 39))
 (segment (start 151.9951 72.78) (end 152.6301 73.415) (width 0.25) (layer "F.Cu") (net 39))
 (segment (start 151.9951 71.51) (end 152.6301 72.145) (width 0.25) (layer "F.Cu") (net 40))
 (segment (start 152.6301 72.145) (end 156.2815 72.145) (width 0.25) (layer "F.Cu") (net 40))
 (segment (start 150.62 71.51) (end 151.9951 71.51) (width 0.25) (layer "F.Cu") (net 40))
 (segment (start 151.9951 70.24) (end 152.6301 70.875) (width 0.25) (layer "F.Cu") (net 41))
 (segment (start 150.62 70.24) (end 151.9951 70.24) (width 0.25) (layer "F.Cu") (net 41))
 (segment (start 152.6301 70.875) (end 156.2815 70.875) (width 0.25) (layer "F.Cu") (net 41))
 (segment (start 152.6301 69.605) (end 156.2815 69.605) (width 0.25) (layer "F.Cu") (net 42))
 (segment (start 150.62 68.97) (end 151.9951 68.97) (width 0.25) (layer "F.Cu") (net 42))
 (segment (start 151.9951 68.97) (end 152.6301 69.605) (width 0.25) (layer "F.Cu") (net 42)))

